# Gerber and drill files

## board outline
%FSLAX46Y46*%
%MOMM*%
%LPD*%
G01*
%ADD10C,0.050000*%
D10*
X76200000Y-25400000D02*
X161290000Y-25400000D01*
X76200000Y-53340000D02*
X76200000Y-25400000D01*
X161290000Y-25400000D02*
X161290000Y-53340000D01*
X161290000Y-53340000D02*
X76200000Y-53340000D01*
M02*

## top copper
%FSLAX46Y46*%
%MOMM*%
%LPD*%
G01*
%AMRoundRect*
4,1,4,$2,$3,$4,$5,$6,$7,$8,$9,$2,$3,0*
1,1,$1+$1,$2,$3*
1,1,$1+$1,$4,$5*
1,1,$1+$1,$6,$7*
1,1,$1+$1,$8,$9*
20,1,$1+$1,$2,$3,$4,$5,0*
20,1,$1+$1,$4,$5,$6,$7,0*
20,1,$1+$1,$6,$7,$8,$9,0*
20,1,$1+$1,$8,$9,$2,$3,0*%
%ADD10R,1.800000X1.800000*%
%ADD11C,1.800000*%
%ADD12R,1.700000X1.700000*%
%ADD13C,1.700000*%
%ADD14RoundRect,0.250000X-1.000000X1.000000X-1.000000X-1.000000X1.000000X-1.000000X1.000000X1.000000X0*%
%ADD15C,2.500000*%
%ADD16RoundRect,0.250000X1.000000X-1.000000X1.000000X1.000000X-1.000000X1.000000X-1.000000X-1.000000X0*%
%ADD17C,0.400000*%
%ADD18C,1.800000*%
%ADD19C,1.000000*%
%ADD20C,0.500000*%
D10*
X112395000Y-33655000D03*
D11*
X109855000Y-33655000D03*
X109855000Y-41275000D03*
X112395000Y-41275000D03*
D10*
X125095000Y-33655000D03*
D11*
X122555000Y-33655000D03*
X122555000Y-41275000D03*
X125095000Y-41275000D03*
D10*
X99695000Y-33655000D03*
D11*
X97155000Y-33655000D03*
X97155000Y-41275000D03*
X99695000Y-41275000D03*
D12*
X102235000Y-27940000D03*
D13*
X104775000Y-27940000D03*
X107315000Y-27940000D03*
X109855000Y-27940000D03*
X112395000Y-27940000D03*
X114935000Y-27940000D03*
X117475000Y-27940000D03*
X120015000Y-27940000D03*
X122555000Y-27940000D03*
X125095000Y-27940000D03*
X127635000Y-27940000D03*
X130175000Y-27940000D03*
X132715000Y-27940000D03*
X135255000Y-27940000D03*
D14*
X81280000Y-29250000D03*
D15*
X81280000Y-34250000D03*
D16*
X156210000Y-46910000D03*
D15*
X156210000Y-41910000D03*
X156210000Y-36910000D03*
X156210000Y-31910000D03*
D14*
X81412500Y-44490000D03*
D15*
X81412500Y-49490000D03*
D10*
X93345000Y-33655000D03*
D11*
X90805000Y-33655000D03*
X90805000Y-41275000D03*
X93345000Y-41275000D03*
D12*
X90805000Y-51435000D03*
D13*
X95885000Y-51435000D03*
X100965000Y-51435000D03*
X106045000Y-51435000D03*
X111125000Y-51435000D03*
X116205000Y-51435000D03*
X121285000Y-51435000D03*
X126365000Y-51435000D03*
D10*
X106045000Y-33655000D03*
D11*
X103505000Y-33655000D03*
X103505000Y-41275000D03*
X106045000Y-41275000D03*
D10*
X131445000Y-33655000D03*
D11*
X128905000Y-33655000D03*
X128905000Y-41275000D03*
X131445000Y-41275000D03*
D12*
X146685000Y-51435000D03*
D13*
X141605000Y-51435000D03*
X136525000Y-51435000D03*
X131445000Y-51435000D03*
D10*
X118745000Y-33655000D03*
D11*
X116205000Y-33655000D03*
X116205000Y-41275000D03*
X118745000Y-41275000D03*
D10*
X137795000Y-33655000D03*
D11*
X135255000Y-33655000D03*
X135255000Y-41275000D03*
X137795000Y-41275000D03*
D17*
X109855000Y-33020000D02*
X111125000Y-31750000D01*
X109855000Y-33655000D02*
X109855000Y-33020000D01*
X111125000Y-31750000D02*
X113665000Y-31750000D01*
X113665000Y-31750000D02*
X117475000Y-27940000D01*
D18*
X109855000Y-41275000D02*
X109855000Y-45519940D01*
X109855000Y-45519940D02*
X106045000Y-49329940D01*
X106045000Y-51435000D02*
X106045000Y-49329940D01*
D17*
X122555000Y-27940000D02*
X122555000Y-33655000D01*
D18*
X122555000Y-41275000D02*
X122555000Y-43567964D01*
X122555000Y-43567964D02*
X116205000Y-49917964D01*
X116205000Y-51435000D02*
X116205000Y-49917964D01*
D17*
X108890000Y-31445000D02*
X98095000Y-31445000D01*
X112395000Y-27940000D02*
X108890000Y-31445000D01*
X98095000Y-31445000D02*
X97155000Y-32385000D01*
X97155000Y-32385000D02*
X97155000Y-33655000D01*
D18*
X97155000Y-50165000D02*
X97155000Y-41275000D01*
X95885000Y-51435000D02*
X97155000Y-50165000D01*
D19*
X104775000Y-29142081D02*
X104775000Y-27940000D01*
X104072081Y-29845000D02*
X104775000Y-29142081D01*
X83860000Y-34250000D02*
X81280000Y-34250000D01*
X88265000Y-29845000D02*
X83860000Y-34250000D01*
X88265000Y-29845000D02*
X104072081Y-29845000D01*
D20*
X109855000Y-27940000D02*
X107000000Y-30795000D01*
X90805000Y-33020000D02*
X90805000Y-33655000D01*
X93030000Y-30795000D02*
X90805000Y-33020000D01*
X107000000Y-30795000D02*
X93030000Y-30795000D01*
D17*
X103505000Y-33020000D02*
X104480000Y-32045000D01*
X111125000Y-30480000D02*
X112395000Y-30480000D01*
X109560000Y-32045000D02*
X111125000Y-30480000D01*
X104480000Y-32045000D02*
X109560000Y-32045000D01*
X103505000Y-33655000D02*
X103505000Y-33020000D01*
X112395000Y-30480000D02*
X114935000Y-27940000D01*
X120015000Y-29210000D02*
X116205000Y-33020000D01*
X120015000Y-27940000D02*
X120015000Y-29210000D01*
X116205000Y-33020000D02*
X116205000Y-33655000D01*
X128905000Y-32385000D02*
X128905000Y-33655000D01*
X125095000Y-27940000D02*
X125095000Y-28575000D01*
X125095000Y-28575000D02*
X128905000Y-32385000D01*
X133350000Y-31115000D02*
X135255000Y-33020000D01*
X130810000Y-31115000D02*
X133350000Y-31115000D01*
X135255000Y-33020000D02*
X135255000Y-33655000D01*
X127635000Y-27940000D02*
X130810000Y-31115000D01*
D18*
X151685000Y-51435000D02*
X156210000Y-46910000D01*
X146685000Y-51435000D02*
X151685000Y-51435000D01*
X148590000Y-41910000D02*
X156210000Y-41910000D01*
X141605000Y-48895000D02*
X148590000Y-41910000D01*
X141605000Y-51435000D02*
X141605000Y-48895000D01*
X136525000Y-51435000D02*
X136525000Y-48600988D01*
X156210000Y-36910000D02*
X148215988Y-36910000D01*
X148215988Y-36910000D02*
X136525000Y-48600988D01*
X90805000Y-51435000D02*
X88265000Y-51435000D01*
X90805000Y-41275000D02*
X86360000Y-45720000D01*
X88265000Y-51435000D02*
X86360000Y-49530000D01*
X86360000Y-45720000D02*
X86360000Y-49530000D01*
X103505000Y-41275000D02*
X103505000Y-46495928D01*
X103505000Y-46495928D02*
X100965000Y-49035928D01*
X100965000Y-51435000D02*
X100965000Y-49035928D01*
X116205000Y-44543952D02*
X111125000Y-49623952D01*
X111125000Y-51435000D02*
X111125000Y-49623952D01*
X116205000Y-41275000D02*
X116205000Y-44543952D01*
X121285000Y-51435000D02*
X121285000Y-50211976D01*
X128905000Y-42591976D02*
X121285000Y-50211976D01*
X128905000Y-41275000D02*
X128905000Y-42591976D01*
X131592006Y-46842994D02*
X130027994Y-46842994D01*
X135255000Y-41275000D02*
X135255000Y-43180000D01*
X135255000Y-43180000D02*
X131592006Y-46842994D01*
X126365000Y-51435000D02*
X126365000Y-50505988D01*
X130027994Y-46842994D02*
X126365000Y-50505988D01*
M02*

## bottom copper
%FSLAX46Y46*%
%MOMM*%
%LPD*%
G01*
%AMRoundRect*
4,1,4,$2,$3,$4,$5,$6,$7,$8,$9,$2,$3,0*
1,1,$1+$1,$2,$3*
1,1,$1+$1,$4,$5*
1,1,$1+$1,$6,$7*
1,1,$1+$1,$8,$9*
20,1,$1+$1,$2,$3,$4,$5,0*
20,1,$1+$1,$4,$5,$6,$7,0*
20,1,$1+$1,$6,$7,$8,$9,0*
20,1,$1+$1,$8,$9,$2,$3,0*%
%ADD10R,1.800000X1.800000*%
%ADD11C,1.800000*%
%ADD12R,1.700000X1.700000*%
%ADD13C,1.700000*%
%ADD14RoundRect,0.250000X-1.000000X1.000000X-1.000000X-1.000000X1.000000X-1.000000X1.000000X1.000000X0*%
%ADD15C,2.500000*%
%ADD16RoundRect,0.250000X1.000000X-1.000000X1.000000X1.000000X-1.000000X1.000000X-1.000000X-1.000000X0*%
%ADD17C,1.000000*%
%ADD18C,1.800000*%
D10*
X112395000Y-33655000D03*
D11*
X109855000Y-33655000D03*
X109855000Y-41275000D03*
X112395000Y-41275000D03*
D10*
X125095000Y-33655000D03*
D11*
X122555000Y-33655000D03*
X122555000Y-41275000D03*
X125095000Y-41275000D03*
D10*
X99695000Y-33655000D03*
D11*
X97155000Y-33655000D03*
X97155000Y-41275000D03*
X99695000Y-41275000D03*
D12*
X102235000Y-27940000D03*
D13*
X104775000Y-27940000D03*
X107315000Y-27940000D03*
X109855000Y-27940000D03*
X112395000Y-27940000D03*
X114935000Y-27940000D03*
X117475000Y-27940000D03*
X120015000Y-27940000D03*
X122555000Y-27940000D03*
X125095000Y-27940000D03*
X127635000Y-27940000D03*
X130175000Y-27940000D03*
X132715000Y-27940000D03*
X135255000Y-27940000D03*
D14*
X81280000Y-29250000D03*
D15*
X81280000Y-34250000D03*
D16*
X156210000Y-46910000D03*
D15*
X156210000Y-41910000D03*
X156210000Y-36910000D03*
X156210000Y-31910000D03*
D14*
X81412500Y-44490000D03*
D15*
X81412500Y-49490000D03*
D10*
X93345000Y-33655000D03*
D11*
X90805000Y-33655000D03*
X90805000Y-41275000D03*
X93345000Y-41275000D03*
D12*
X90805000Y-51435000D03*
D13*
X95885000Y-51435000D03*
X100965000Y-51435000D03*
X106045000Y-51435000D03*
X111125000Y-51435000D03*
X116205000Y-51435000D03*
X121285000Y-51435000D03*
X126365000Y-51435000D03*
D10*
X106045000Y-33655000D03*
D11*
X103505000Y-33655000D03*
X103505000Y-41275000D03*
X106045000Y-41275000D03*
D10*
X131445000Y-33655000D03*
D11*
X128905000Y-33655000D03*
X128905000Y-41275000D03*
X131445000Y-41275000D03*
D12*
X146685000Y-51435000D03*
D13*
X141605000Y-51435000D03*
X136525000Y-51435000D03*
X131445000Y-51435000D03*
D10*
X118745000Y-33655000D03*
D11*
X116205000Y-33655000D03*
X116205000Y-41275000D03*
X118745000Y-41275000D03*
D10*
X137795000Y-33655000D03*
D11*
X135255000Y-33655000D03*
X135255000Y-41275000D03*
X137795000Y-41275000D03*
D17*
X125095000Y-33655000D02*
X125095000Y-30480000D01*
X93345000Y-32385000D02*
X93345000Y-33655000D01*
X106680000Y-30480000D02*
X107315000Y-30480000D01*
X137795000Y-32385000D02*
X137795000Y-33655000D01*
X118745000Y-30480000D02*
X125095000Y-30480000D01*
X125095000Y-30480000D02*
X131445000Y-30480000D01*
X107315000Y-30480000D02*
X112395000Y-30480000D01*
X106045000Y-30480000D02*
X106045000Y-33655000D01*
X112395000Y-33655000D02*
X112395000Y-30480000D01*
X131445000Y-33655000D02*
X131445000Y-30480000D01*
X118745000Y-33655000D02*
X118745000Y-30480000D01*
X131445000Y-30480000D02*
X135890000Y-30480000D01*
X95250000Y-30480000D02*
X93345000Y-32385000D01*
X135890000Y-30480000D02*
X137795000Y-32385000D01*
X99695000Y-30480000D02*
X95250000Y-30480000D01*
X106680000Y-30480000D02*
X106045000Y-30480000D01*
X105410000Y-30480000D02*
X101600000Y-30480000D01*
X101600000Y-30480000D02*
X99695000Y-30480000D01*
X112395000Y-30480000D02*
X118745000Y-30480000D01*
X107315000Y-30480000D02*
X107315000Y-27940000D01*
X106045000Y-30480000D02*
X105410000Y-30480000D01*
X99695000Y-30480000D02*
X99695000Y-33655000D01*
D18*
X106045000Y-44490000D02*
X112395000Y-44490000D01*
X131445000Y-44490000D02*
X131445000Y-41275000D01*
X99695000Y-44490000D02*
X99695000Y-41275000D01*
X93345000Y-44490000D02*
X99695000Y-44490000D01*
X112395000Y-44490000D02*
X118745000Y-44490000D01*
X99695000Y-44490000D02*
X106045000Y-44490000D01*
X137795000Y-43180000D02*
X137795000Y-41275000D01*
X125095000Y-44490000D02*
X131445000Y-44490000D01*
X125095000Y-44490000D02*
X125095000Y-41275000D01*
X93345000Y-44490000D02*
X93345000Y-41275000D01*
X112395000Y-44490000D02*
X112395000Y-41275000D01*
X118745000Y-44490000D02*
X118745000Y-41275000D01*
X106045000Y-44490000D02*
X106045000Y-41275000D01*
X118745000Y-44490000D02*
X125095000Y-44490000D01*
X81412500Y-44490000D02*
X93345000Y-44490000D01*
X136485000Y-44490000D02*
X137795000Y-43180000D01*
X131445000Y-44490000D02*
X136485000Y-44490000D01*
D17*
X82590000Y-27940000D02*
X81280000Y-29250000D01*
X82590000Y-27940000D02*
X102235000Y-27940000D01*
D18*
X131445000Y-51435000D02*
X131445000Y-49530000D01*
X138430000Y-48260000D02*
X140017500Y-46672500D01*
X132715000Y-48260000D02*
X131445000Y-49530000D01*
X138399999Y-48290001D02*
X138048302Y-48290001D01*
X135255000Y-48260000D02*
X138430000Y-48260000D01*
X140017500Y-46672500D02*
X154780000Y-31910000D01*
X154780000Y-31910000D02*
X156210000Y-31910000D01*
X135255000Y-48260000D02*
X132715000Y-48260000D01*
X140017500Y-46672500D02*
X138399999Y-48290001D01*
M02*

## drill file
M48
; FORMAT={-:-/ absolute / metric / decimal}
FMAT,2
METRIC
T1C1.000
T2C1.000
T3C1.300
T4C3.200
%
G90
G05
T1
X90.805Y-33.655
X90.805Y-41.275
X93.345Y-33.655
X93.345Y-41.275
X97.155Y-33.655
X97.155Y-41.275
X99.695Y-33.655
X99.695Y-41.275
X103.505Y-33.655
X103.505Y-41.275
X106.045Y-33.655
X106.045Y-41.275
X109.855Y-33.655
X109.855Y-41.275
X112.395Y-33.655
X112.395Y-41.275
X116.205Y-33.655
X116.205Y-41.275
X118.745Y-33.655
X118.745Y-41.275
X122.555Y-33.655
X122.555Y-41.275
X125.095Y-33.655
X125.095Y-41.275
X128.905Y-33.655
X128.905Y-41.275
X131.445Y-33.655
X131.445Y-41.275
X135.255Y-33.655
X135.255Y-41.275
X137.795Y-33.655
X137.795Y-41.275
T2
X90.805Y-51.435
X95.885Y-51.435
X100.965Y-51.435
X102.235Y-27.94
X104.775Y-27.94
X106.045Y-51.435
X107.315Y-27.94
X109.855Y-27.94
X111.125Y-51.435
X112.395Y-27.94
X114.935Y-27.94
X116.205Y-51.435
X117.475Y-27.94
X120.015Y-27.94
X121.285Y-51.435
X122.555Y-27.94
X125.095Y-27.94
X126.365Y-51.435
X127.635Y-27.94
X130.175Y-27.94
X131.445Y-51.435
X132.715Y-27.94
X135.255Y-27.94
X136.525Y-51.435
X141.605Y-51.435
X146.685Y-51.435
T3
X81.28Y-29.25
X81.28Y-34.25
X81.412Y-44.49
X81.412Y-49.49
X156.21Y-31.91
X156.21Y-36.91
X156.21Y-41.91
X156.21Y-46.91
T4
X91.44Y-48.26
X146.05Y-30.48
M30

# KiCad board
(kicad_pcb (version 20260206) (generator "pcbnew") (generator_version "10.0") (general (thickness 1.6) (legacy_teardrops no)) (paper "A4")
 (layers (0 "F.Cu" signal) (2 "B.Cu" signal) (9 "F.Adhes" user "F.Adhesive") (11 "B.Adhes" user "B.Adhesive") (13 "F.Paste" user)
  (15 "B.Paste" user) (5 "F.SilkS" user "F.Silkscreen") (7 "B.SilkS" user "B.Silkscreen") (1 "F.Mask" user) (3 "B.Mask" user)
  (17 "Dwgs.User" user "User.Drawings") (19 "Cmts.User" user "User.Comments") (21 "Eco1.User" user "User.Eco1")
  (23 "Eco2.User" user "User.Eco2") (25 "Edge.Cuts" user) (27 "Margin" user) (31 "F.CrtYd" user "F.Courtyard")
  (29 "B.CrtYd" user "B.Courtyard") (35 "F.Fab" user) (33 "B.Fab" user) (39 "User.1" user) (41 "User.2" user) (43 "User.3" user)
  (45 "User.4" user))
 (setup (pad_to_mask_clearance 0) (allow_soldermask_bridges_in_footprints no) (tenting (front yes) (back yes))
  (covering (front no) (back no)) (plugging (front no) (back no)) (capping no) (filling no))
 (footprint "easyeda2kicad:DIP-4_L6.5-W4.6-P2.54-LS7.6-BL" (layer "F.Cu") (at 111.125 37.465 180)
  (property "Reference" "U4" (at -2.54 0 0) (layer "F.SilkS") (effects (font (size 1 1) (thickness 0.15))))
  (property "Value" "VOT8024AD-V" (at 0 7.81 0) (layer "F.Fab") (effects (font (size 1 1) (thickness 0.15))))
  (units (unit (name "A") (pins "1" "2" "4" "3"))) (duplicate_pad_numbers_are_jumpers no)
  (pad "1" thru_hole rect (at -1.27 3.81) (size 1.8 1.8) (drill 0.999998) (layers "*.Cu" "*.Mask") (remove_unused_layers no) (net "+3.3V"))
  (pad "2" thru_hole circle (at 1.27 3.81 270) (size 1.8 1.8) (drill 0.999998) (layers "*.Cu" "*.Mask") (remove_unused_layers no)
   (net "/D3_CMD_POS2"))
  (pad "3" thru_hole circle (at 1.27 -3.81 270) (size 1.8 1.8) (drill 0.999998) (layers "*.Cu" "*.Mask") (remove_unused_layers no)
   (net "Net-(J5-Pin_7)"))
  (pad "4" thru_hole circle (at -1.27 -3.81 270) (size 1.8 1.8) (drill 0.999998) (layers "*.Cu" "*.Mask") (remove_unused_layers no)
   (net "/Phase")))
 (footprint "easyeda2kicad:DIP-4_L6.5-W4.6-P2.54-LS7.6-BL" (layer "F.Cu") (at 123.825 37.465 180)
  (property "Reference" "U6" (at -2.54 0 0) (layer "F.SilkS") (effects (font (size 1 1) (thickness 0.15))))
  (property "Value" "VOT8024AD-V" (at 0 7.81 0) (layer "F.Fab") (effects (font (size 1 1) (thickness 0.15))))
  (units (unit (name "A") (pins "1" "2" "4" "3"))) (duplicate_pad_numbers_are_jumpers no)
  (pad "1" thru_hole rect (at -1.27 3.81) (size 1.8 1.8) (drill 0.999998) (layers "*.Cu" "*.Mask") (remove_unused_layers no) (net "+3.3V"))
  (pad "2" thru_hole circle (at 1.27 3.81 270) (size 1.8 1.8) (drill 0.999998) (layers "*.Cu" "*.Mask") (remove_unused_layers no)
   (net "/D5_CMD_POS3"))
  (pad "3" thru_hole circle (at 1.27 -3.81 270) (size 1.8 1.8) (drill 0.999998) (layers "*.Cu" "*.Mask") (remove_unused_layers no)
   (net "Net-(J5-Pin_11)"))
  (pad "4" thru_hole circle (at -1.27 -3.81 270) (size 1.8 1.8) (drill 0.999998) (layers "*.Cu" "*.Mask") (remove_unused_layers no)
   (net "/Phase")))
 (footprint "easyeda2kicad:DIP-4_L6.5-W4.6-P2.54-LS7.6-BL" (layer "F.Cu") (at 98.425 37.465 180)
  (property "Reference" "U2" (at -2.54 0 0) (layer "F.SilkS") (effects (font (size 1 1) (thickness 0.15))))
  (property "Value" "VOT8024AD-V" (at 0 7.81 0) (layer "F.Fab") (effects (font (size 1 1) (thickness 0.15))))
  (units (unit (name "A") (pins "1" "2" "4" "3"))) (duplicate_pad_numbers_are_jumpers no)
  (pad "1" thru_hole rect (at -1.27 3.81) (size 1.8 1.8) (drill 0.999998) (layers "*.Cu" "*.Mask") (remove_unused_layers no) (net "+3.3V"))
  (pad "2" thru_hole circle (at 1.27 3.81 270) (size 1.8 1.8) (drill 0.999998) (layers "*.Cu" "*.Mask") (remove_unused_layers no)
   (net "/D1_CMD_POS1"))
  (pad "3" thru_hole circle (at 1.27 -3.81 270) (size 1.8 1.8) (drill 0.999998) (layers "*.Cu" "*.Mask") (remove_unused_layers no)
   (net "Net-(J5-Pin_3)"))
  (pad "4" thru_hole circle (at -1.27 -3.81 270) (size 1.8 1.8) (drill 0.999998) (layers "*.Cu" "*.Mask") (remove_unused_layers no)
   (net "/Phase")))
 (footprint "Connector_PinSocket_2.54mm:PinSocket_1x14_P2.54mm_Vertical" (layer "F.Cu") (at 102.235 27.94 90)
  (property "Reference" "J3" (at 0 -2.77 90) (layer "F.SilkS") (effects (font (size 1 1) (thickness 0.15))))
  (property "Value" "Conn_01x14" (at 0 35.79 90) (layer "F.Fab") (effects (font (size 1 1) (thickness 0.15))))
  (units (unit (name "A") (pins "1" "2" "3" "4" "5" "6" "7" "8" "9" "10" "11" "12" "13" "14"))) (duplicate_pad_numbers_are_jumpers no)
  (pad "1" thru_hole rect (at 0 0 90) (size 1.7 1.7) (drill 1) (layers "*.Cu" "*.Mask") (remove_unused_layers no) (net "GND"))
  (pad "2" thru_hole circle (at 0 2.54 90) (size 1.7 1.7) (drill 1) (layers "*.Cu" "*.Mask") (remove_unused_layers no) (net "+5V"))
  (pad "3" thru_hole circle (at 0 5.08 90) (size 1.7 1.7) (drill 1) (layers "*.Cu" "*.Mask") (remove_unused_layers no) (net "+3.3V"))
  (pad "4" thru_hole circle (at 0 7.62 90) (size 1.7 1.7) (drill 1) (layers "*.Cu" "*.Mask") (remove_unused_layers no) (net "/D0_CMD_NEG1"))
  (pad "5" thru_hole circle (at 0 10.16 90) (size 1.7 1.7) (drill 1) (layers "*.Cu" "*.Mask") (remove_unused_layers no) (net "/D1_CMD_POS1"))
  (pad "6" thru_hole circle (at 0 12.7 90) (size 1.7 1.7) (drill 1) (layers "*.Cu" "*.Mask") (remove_unused_layers no) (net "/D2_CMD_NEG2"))
  (pad "7" thru_hole circle (at 0 15.24 90) (size 1.7 1.7) (drill 1) (layers "*.Cu" "*.Mask") (remove_unused_layers no) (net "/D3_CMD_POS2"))
  (pad "8" thru_hole circle (at 0 17.78 90) (size 1.7 1.7) (drill 1) (layers "*.Cu" "*.Mask") (remove_unused_layers no) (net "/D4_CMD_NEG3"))
  (pad "9" thru_hole circle (at 0 20.32 90) (size 1.7 1.7) (drill 1) (layers "*.Cu" "*.Mask") (remove_unused_layers no) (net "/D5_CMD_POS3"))
  (pad "10" thru_hole circle (at 0 22.86 90) (size 1.7 1.7) (drill 1) (layers "*.Cu" "*.Mask") (remove_unused_layers no)
   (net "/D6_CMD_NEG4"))
  (pad "11" thru_hole circle (at 0 25.4 90) (size 1.7 1.7) (drill 1) (layers "*.Cu" "*.Mask") (remove_unused_layers no) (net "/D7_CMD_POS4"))
  (pad "12" thru_hole circle (at 0 27.94 90) (size 1.7 1.7) (drill 1) (layers "*.Cu" "*.Mask") (remove_unused_layers no)
   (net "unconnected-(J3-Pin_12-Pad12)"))
  (pad "13" thru_hole circle (at 0 30.48 90) (size 1.7 1.7) (drill 1) (layers "*.Cu" "*.Mask") (remove_unused_layers no)
   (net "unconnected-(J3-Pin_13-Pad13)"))
  (pad "14" thru_hole circle (at 0 33.02 90) (size 1.7 1.7) (drill 1) (layers "*.Cu" "*.Mask") (remove_unused_layers no)
   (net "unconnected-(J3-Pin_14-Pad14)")))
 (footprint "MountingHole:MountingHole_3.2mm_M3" (layer "F.Cu") (at 91.44 48.26)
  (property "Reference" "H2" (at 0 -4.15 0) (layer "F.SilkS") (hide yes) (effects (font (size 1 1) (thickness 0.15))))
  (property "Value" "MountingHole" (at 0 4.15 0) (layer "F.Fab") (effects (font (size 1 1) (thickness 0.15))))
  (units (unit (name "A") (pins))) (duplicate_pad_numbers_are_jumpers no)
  (pad "" np_thru_hole circle (at 0 0) (size 3.2 3.2) (drill 3.2) (layers "*.Cu" "*.Mask")))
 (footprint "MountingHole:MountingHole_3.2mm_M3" (layer "F.Cu") (at 146.05 30.48)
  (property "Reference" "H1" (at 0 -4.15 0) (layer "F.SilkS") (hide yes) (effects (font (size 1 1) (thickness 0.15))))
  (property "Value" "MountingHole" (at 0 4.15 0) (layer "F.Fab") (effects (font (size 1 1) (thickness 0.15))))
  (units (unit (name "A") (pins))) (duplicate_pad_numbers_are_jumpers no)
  (pad "" np_thru_hole circle (at 0 0) (size 3.2 3.2) (drill 3.2) (layers "*.Cu" "*.Mask")))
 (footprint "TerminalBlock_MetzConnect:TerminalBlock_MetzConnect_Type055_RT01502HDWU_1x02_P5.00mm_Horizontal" (layer "F.Cu")
  (at 81.28 29.25 -90)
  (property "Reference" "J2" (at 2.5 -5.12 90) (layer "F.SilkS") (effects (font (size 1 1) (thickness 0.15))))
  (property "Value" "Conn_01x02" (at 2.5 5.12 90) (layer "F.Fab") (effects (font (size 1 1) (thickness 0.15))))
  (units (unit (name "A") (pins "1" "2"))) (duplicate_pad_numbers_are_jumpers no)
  (pad "1" thru_hole roundrect (at 0 0 270) (size 2.5 2.5) (drill 1.3) (layers "*.Cu" "*.Mask") (remove_unused_layers no)
   (roundrect_rratio 0.1) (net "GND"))
  (pad "2" thru_hole circle (at 5 0 270) (size 2.5 2.5) (drill 1.3) (layers "*.Cu" "*.Mask") (remove_unused_layers no) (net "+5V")))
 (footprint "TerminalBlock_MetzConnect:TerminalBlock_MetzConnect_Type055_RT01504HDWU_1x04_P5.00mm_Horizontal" (layer "F.Cu")
  (at 156.21 46.91 90)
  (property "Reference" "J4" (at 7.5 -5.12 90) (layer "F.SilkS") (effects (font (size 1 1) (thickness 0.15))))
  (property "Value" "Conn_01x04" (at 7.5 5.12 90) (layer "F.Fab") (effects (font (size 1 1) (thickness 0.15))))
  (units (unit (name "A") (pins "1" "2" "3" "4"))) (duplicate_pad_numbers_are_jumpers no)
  (pad "1" thru_hole roundrect (at 0 0 90) (size 2.5 2.5) (drill 1.3) (layers "*.Cu" "*.Mask") (remove_unused_layers no)
   (roundrect_rratio 0.1) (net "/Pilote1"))
  (pad "2" thru_hole circle (at 5 0 90) (size 2.5 2.5) (drill 1.3) (layers "*.Cu" "*.Mask") (remove_unused_layers no) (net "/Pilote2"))
  (pad "3" thru_hole circle (at 10 0 90) (size 2.5 2.5) (drill 1.3) (layers "*.Cu" "*.Mask") (remove_unused_layers no) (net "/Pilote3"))
  (pad "4" thru_hole circle (at 15 0 90) (size 2.5 2.5) (drill 1.3) (layers "*.Cu" "*.Mask") (remove_unused_layers no) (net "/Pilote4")))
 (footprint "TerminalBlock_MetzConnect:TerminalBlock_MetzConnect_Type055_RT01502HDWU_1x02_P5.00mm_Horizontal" (layer "F.Cu")
  (at 81.4125 44.49 -90)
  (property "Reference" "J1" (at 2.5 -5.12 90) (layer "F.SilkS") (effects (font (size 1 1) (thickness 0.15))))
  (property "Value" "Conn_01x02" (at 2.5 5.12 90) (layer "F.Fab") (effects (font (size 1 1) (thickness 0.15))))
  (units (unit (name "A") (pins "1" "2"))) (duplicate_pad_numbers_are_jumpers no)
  (pad "1" thru_hole roundrect (at 0 0 270) (size 2.5 2.5) (drill 1.3) (layers "*.Cu" "*.Mask") (remove_unused_layers no)
   (roundrect_rratio 0.1) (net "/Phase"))
  (pad "2" thru_hole circle (at 5 0 270) (size 2.5 2.5) (drill 1.3) (layers "*.Cu" "*.Mask") (remove_unused_layers no)
   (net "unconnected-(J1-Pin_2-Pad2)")))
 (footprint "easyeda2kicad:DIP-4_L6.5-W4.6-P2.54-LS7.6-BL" (layer "F.Cu") (at 92.075 37.465 180)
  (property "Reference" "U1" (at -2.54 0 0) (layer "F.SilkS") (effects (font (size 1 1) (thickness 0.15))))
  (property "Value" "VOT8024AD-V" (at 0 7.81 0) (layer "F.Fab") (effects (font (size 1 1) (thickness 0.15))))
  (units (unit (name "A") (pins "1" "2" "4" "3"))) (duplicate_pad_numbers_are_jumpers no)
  (pad "1" thru_hole rect (at -1.27 3.81) (size 1.8 1.8) (drill 0.999998) (layers "*.Cu" "*.Mask") (remove_unused_layers no) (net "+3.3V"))
  (pad "2" thru_hole circle (at 1.27 3.81 270) (size 1.8 1.8) (drill 0.999998) (layers "*.Cu" "*.Mask") (remove_unused_layers no)
   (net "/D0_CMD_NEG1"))
  (pad "3" thru_hole circle (at 1.27 -3.81 270) (size 1.8 1.8) (drill 0.999998) (layers "*.Cu" "*.Mask") (remove_unused_layers no)
   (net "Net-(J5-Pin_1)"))
  (pad "4" thru_hole circle (at -1.27 -3.81 270) (size 1.8 1.8) (drill 0.999998) (layers "*.Cu" "*.Mask") (remove_unused_layers no)
   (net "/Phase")))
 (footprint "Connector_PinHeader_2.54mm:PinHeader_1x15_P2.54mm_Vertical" (layer "F.Cu") (at 90.805 51.435 90)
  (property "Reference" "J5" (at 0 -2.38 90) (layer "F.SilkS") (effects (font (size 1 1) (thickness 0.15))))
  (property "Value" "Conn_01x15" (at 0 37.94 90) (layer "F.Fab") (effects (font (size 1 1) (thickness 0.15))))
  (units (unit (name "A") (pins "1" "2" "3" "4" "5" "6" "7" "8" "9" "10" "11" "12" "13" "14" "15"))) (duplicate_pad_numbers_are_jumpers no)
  (pad "1" thru_hole rect (at 0 0 90) (size 1.7 1.7) (drill 1) (layers "*.Cu" "*.Mask") (remove_unused_layers no) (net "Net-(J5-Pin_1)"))
  (pad "3" thru_hole circle (at 0 5.08 90) (size 1.7 1.7) (drill 1) (layers "*.Cu" "*.Mask") (remove_unused_layers no)
   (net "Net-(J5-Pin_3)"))
  (pad "5" thru_hole circle (at 0 10.16 90) (size 1.7 1.7) (drill 1) (layers "*.Cu" "*.Mask") (remove_unused_layers no)
   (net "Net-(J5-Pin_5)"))
  (pad "7" thru_hole circle (at 0 15.24 90) (size 1.7 1.7) (drill 1) (layers "*.Cu" "*.Mask") (remove_unused_layers no)
   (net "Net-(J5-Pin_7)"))
  (pad "9" thru_hole circle (at 0 20.32 90) (size 1.7 1.7) (drill 1) (layers "*.Cu" "*.Mask") (remove_unused_layers no)
   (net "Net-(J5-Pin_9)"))
  (pad "11" thru_hole circle (at 0 25.4 90) (size 1.7 1.7) (drill 1) (layers "*.Cu" "*.Mask") (remove_unused_layers no)
   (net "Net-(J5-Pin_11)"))
  (pad "13" thru_hole circle (at 0 30.48 90) (size 1.7 1.7) (drill 1) (layers "*.Cu" "*.Mask") (remove_unused_layers no)
   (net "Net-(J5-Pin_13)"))
  (pad "15" thru_hole circle (at 0 35.56 90) (size 1.7 1.7) (drill 1) (layers "*.Cu" "*.Mask") (remove_unused_layers no)
   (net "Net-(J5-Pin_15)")))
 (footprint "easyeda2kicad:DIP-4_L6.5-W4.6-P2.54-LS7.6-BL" (layer "F.Cu") (at 104.775 37.465 180)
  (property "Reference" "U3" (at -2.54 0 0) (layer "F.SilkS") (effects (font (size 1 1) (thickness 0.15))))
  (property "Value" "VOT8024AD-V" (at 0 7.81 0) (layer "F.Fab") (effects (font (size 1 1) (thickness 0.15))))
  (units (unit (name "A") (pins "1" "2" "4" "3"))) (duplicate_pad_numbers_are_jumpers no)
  (pad "1" thru_hole rect (at -1.27 3.81) (size 1.8 1.8) (drill 0.999998) (layers "*.Cu" "*.Mask") (remove_unused_layers no) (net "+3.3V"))
  (pad "2" thru_hole circle (at 1.27 3.81 270) (size 1.8 1.8) (drill 0.999998) (layers "*.Cu" "*.Mask") (remove_unused_layers no)
   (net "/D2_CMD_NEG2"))
  (pad "3" thru_hole circle (at 1.27 -3.81 270) (size 1.8 1.8) (drill 0.999998) (layers "*.Cu" "*.Mask") (remove_unused_layers no)
   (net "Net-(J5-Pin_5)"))
  (pad "4" thru_hole circle (at -1.27 -3.81 270) (size 1.8 1.8) (drill 0.999998) (layers "*.Cu" "*.Mask") (remove_unused_layers no)
   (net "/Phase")))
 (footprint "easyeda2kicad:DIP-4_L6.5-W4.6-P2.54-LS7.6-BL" (layer "F.Cu") (at 130.175 37.465 180)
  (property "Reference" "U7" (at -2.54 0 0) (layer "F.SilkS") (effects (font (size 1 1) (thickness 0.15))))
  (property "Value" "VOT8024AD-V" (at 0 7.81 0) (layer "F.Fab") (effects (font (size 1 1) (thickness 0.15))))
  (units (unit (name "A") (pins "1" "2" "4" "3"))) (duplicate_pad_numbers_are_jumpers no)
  (pad "1" thru_hole rect (at -1.27 3.81) (size 1.8 1.8) (drill 0.999998) (layers "*.Cu" "*.Mask") (remove_unused_layers no) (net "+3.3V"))
  (pad "2" thru_hole circle (at 1.27 3.81 270) (size 1.8 1.8) (drill 0.999998) (layers "*.Cu" "*.Mask") (remove_unused_layers no)
   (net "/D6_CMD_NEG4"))
  (pad "3" thru_hole circle (at 1.27 -3.81 270) (size 1.8 1.8) (drill 0.999998) (layers "*.Cu" "*.Mask") (remove_unused_layers no)
   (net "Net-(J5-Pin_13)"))
  (pad "4" thru_hole circle (at -1.27 -3.81 270) (size 1.8 1.8) (drill 0.999998) (layers "*.Cu" "*.Mask") (remove_unused_layers no)
   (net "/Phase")))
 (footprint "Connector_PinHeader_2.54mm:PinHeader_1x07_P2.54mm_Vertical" (layer "F.Cu") (at 146.685 51.435 -90)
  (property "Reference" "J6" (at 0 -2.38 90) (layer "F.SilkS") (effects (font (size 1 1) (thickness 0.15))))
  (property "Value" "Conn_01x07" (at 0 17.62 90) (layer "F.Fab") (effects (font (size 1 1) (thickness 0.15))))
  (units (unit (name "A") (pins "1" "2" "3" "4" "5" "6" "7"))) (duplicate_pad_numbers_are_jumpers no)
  (pad "1" thru_hole rect (at 0 0 270) (size 1.7 1.7) (drill 1) (layers "*.Cu" "*.Mask") (remove_unused_layers no) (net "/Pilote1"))
  (pad "3" thru_hole circle (at 0 5.08 270) (size 1.7 1.7) (drill 1) (layers "*.Cu" "*.Mask") (remove_unused_layers no) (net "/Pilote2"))
  (pad "5" thru_hole circle (at 0 10.16 270) (size 1.7 1.7) (drill 1) (layers "*.Cu" "*.Mask") (remove_unused_layers no) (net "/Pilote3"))
  (pad "7" thru_hole circle (at 0 15.24 270) (size 1.7 1.7) (drill 1) (layers "*.Cu" "*.Mask") (remove_unused_layers no) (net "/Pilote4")))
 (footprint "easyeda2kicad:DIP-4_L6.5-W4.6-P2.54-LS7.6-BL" (layer "F.Cu") (at 117.475 37.465 180)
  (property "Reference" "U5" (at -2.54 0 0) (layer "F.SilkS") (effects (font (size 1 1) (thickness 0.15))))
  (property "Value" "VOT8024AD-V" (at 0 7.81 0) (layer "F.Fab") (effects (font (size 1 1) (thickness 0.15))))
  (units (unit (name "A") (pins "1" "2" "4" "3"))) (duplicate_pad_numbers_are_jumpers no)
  (pad "1" thru_hole rect (at -1.27 3.81) (size 1.8 1.8) (drill 0.999998) (layers "*.Cu" "*.Mask") (remove_unused_layers no) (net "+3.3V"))
  (pad "2" thru_hole circle (at 1.27 3.81 270) (size 1.8 1.8) (drill 0.999998) (layers "*.Cu" "*.Mask") (remove_unused_layers no)
   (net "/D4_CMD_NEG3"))
  (pad "3" thru_hole circle (at 1.27 -3.81 270) (size 1.8 1.8) (drill 0.999998) (layers "*.Cu" "*.Mask") (remove_unused_layers no)
   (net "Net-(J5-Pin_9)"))
  (pad "4" thru_hole circle (at -1.27 -3.81 270) (size 1.8 1.8) (drill 0.999998) (layers "*.Cu" "*.Mask") (remove_unused_layers no)
   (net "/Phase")))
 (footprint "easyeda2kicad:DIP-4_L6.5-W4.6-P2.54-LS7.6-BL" (layer "F.Cu") (at 136.525 37.465 180)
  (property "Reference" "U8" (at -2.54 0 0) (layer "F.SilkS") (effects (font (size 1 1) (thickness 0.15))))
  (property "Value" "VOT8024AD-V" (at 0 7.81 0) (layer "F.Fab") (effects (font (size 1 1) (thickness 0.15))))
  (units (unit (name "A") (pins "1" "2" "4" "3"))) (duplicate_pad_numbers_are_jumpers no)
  (pad "1" thru_hole rect (at -1.27 3.81) (size 1.8 1.8) (drill 0.999998) (layers "*.Cu" "*.Mask") (remove_unused_layers no) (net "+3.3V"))
  (pad "2" thru_hole circle (at 1.27 3.81 270) (size 1.8 1.8) (drill 0.999998) (layers "*.Cu" "*.Mask") (remove_unused_layers no)
   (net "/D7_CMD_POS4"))
  (pad "3" thru_hole circle (at 1.27 -3.81 270) (size 1.8 1.8) (drill 0.999998) (layers "*.Cu" "*.Mask") (remove_unused_layers no)
   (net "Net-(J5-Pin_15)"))
  (pad "4" thru_hole circle (at -1.27 -3.81 270) (size 1.8 1.8) (drill 0.999998) (layers "*.Cu" "*.Mask") (remove_unused_layers no)
   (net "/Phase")))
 (gr_line (start 76.2 25.4) (end 161.29 25.4) (stroke (width 0.05) (type default)) (layer "Edge.Cuts"))
 (gr_line (start 76.2 53.34) (end 76.2 25.4) (stroke (width 0.05) (type default)) (layer "Edge.Cuts"))
 (gr_line (start 161.29 25.4) (end 161.29 53.34) (stroke (width 0.05) (type default)) (layer "Edge.Cuts"))
 (gr_line (start 161.29 53.34) (end 76.2 53.34) (stroke (width 0.05) (type default)) (layer "Edge.Cuts"))
 (segment (start 125.095 33.655) (end 125.095 30.48) (width 1) (layer "B.Cu") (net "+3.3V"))
 (segment (start 93.345 32.385) (end 93.345 33.655) (width 1) (layer "B.Cu") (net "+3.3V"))
 (segment (start 106.68 30.48) (end 107.315 30.48) (width 1) (layer "B.Cu") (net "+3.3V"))
 (segment (start 137.795 32.385) (end 137.795 33.655) (width 1) (layer "B.Cu") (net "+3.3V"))
 (segment (start 118.745 30.48) (end 125.095 30.48) (width 1) (layer "B.Cu") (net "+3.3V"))
 (segment (start 125.095 30.48) (end 131.445 30.48) (width 1) (layer "B.Cu") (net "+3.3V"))
 (segment (start 107.315 30.48) (end 112.395 30.48) (width 1) (layer "B.Cu") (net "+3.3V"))
 (segment (start 106.045 30.48) (end 106.045 33.655) (width 1) (layer "B.Cu") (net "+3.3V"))
 (segment (start 112.395 33.655) (end 112.395 30.48) (width 1) (layer "B.Cu") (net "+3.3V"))
 (segment (start 131.445 33.655) (end 131.445 30.48) (width 1) (layer "B.Cu") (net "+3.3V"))
 (segment (start 118.745 33.655) (end 118.745 30.48) (width 1) (layer "B.Cu") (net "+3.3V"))
 (segment (start 131.445 30.48) (end 135.89 30.48) (width 1) (layer "B.Cu") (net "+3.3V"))
 (segment (start 95.25 30.48) (end 93.345 32.385) (width 1) (layer "B.Cu") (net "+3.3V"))
 (segment (start 135.89 30.48) (end 137.795 32.385) (width 1) (layer "B.Cu") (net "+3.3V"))
 (segment (start 99.695 30.48) (end 95.25 30.48) (width 1) (layer "B.Cu") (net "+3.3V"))
 (segment (start 106.68 30.48) (end 106.045 30.48) (width 1) (layer "B.Cu") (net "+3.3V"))
 (segment (start 105.41 30.48) (end 101.6 30.48) (width 1) (layer "B.Cu") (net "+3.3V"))
 (segment (start 101.6 30.48) (end 99.695 30.48) (width 1) (layer "B.Cu") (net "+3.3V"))
 (segment (start 112.395 30.48) (end 118.745 30.48) (width 1) (layer "B.Cu") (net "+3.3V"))
 (segment (start 107.315 30.48) (end 107.315 27.94) (width 1) (layer "B.Cu") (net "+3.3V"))
 (segment (start 106.045 30.48) (end 105.41 30.48) (width 1) (layer "B.Cu") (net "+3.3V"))
 (segment (start 99.695 30.48) (end 99.695 33.655) (width 1) (layer "B.Cu") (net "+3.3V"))
 (segment (start 109.855 33.02) (end 111.125 31.75) (width 0.4) (layer "F.Cu") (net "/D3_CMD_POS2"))
 (segment (start 109.855 33.655) (end 109.855 33.02) (width 0.4) (layer "F.Cu") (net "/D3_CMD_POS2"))
 (segment (start 111.125 31.75) (end 113.665 31.75) (width 0.4) (layer "F.Cu") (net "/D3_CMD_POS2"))
 (segment (start 113.665 31.75) (end 117.475 27.94) (width 0.4) (layer "F.Cu") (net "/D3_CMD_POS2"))
 (segment (start 109.855 41.275) (end 109.855 45.51994) (width 1.8) (layer "F.Cu") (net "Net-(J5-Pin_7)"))
 (segment (start 109.855 45.51994) (end 106.045 49.32994) (width 1.8) (layer "F.Cu") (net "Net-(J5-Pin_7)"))
 (segment (start 106.045 51.435) (end 106.045 49.32994) (width 1.8) (layer "F.Cu") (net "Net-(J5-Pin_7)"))
 (segment (start 106.045 44.49) (end 112.395 44.49) (width 1.8) (layer "B.Cu") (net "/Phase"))
 (segment (start 131.445 44.49) (end 131.445 41.275) (width 1.8) (layer "B.Cu") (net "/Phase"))
 (segment (start 99.695 44.49) (end 99.695 41.275) (width 1.8) (layer "B.Cu") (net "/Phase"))
 (segment (start 93.345 44.49) (end 99.695 44.49) (width 1.8) (layer "B.Cu") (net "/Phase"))
 (segment (start 112.395 44.49) (end 118.745 44.49) (width 1.8) (layer "B.Cu") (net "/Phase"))
 (segment (start 99.695 44.49) (end 106.045 44.49) (width 1.8) (layer "B.Cu") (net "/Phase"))
 (segment (start 137.795 43.18) (end 137.795 41.275) (width 1.8) (layer "B.Cu") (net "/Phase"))
 (segment (start 125.095 44.49) (end 131.445 44.49) (width 1.8) (layer "B.Cu") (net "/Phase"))
 (segment (start 125.095 44.49) (end 125.095 41.275) (width 1.8) (layer "B.Cu") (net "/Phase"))
 (segment (start 93.345 44.49) (end 93.345 41.275) (width 1.8) (layer "B.Cu") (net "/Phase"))
 (segment (start 112.395 44.49) (end 112.395 41.275) (width 1.8) (layer "B.Cu") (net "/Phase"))
 (segment (start 118.745 44.49) (end 118.745 41.275) (width 1.8) (layer "B.Cu") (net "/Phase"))
 (segment (start 106.045 44.49) (end 106.045 41.275) (width 1.8) (layer "B.Cu") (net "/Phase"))
 (segment (start 118.745 44.49) (end 125.095 44.49) (width 1.8) (layer "B.Cu") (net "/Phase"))
 (segment (start 81.4125 44.49) (end 93.345 44.49) (width 1.8) (layer "B.Cu") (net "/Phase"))
 (segment (start 136.485 44.49) (end 137.795 43.18) (width 1.8) (layer "B.Cu") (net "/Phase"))
 (segment (start 131.445 44.49) (end 136.485 44.49) (width 1.8) (layer "B.Cu") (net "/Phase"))
 (segment (start 122.555 27.94) (end 122.555 33.655) (width 0.4) (layer "F.Cu") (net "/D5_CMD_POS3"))
 (segment (start 122.555 41.275) (end 122.555 43.567964) (width 1.8) (layer "F.Cu") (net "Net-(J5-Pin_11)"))
 (segment (start 122.555 43.567964) (end 116.205 49.917964) (width 1.8) (layer "F.Cu") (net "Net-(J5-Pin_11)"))
 (segment (start 116.205 51.435) (end 116.205 49.917964) (width 1.8) (layer "F.Cu") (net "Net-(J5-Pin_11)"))
 (segment (start 108.89 31.445) (end 98.095 31.445) (width 0.4) (layer "F.Cu") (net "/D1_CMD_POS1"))
 (segment (start 112.395 27.94) (end 108.89 31.445) (width 0.4) (layer "F.Cu") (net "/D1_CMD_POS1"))
 (segment (start 98.095 31.445) (end 97.155 32.385) (width 0.4) (layer "F.Cu") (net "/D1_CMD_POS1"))
 (segment (start 97.155 32.385) (end 97.155 33.655) (width 0.4) (layer "F.Cu") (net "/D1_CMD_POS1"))
 (segment (start 97.155 50.165) (end 97.155 41.275) (width 1.8) (layer "F.Cu") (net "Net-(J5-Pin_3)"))
 (segment (start 95.885 51.435) (end 97.155 50.165) (width 1.8) (layer "F.Cu") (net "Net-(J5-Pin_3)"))
 (segment (start 82.59 27.94) (end 81.28 29.25) (width 1) (layer "B.Cu") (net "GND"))
 (segment (start 82.59 27.94) (end 102.235 27.94) (width 1) (layer "B.Cu") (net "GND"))
 (segment (start 104.775 29.142081) (end 104.775 27.94) (width 1) (layer "F.Cu") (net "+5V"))
 (segment (start 104.072081 29.845) (end 104.775 29.142081) (width 1) (layer "F.Cu") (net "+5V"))
 (segment (start 83.86 34.25) (end 81.28 34.25) (width 1) (layer "F.Cu") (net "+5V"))
 (segment (start 88.265 29.845) (end 83.86 34.25) (width 1) (layer "F.Cu") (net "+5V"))
 (segment (start 88.265 29.845) (end 104.072081 29.845) (width 1) (layer "F.Cu") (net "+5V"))
 (segment (start 109.855 27.94) (end 107 30.795) (width 0.5) (layer "F.Cu") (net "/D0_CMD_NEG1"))
 (segment (start 90.805 33.02) (end 90.805 33.655) (width 0.5) (layer "F.Cu") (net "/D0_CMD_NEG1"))
 (segment (start 93.03 30.795) (end 90.805 33.02) (width 0.5) (layer "F.Cu") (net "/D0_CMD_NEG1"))
 (segment (start 107 30.795) (end 93.03 30.795) (width 0.5) (layer "F.Cu") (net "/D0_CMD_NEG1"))
 (segment (start 103.505 33.02) (end 104.48 32.045) (width 0.4) (layer "F.Cu") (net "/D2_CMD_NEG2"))
 (segment (start 111.125 30.48) (end 112.395 30.48) (width 0.4) (layer "F.Cu") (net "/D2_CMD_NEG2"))
 (segment (start 109.56 32.045) (end 111.125 30.48) (width 0.4) (layer "F.Cu") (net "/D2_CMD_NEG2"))
 (segment (start 104.48 32.045) (end 109.56 32.045) (width 0.4) (layer "F.Cu") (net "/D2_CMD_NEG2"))
 (segment (start 103.505 33.655) (end 103.505 33.02) (width 0.4) (layer "F.Cu") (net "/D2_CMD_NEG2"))
 (segment (start 112.395 30.48) (end 114.935 27.94) (width 0.4) (layer "F.Cu") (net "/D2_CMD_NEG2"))
 (segment (start 120.015 29.21) (end 116.205 33.02) (width 0.4) (layer "F.Cu") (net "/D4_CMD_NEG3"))
 (segment (start 120.015 27.94) (end 120.015 29.21) (width 0.4) (layer "F.Cu") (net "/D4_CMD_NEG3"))
 (segment (start 116.205 33.02) (end 116.205 33.655) (width 0.4) (layer "F.Cu") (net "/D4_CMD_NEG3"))
 (segment (start 128.905 32.385) (end 128.905 33.655) (width 0.4) (layer "F.Cu") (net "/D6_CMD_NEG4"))
 (segment (start 125.095 27.94) (end 125.095 28.575) (width 0.4) (layer "F.Cu") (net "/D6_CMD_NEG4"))
 (segment (start 125.095 28.575) (end 128.905 32.385) (width 0.4) (layer "F.Cu") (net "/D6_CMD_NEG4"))
 (segment (start 133.35 31.115) (end 135.255 33.02) (width 0.4) (layer "F.Cu") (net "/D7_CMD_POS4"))
 (segment (start 130.81 31.115) (end 133.35 31.115) (width 0.4) (layer "F.Cu") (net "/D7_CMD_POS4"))
 (segment (start 135.255 33.02) (end 135.255 33.655) (width 0.4) (layer "F.Cu") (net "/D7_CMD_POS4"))
 (segment (start 127.635 27.94) (end 130.81 31.115) (width 0.4) (layer "F.Cu") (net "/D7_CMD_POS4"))
 (segment (start 151.685 51.435) (end 156.21 46.91) (width 1.8) (layer "F.Cu") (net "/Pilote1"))
 (segment (start 146.685 51.435) (end 151.685 51.435) (width 1.8) (layer "F.Cu") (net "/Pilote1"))
 (segment (start 148.59 41.91) (end 156.21 41.91) (width 1.8) (layer "F.Cu") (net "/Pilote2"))
 (segment (start 141.605 48.895) (end 148.59 41.91) (width 1.8) (layer "F.Cu") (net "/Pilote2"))
 (segment (start 141.605 51.435) (end 141.605 48.895) (width 1.8) (layer "F.Cu") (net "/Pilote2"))
 (segment (start 136.525 51.435) (end 136.525 48.600988) (width 1.8) (layer "F.Cu") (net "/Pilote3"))
 (segment (start 156.21 36.91) (end 148.215988 36.91) (width 1.8) (layer "F.Cu") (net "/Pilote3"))
 (segment (start 148.215988 36.91) (end 136.525 48.600988) (width 1.8) (layer "F.Cu") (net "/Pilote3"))
 (segment (start 131.445 51.435) (end 131.445 49.53) (width 1.8) (layer "B.Cu") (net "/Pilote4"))
 (segment (start 138.43 48.26) (end 140.0175 46.6725) (width 1.8) (layer "B.Cu") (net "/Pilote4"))
 (segment (start 132.715 48.26) (end 131.445 49.53) (width 1.8) (layer "B.Cu") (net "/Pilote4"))
 (segment (start 138.399999 48.290001) (end 138.048302 48.290001) (width 1.8) (layer "B.Cu") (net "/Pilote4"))
 (segment (start 135.255 48.26) (end 138.43 48.26) (width 1.8) (layer "B.Cu") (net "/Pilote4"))
 (segment (start 140.0175 46.6725) (end 154.78 31.91) (width 1.8) (layer "B.Cu") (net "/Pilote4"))
 (segment (start 154.78 31.91) (end 156.21 31.91) (width 1.8) (layer "B.Cu") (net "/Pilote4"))
 (segment (start 135.255 48.26) (end 132.715 48.26) (width 1.8) (layer "B.Cu") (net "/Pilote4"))
 (segment (start 140.0175 46.6725) (end 138.399999 48.290001) (width 1.8) (layer "B.Cu") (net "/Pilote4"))
 (segment (start 90.805 51.435) (end 88.265 51.435) (width 1.8) (layer "F.Cu") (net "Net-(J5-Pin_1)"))
 (segment (start 90.805 41.275) (end 86.36 45.72) (width 1.8) (layer "F.Cu") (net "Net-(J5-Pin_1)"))
 (segment (start 88.265 51.435) (end 86.36 49.53) (width 1.8) (layer "F.Cu") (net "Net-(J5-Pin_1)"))
 (segment (start 86.36 45.72) (end 86.36 49.53) (width 1.8) (layer "F.Cu") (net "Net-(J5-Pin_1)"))
 (segment (start 103.505 41.275) (end 103.505 46.495928) (width 1.8) (layer "F.Cu") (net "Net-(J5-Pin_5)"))
 (segment (start 103.505 46.495928) (end 100.965 49.035928) (width 1.8) (layer "F.Cu") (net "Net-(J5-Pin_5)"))
 (segment (start 100.965 51.435) (end 100.965 49.035928) (width 1.8) (layer "F.Cu") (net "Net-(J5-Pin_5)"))
 (segment (start 116.205 44.543952) (end 111.125 49.623952) (width 1.8) (layer "F.Cu") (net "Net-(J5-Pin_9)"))
 (segment (start 111.125 51.435) (end 111.125 49.623952) (width 1.8) (layer "F.Cu") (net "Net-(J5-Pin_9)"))
 (segment (start 116.205 41.275) (end 116.205 44.543952) (width 1.8) (layer "F.Cu") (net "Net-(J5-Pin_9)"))
 (segment (start 121.285 51.435) (end 121.285 50.211976) (width 1.8) (layer "F.Cu") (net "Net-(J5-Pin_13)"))
 (segment (start 128.905 42.591976) (end 121.285 50.211976) (width 1.8) (layer "F.Cu") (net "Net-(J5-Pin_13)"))
 (segment (start 128.905 41.275) (end 128.905 42.591976) (width 1.8) (layer "F.Cu") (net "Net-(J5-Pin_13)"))
 (segment (start 131.592006 46.842994) (end 130.027994 46.842994) (width 1.8) (layer "F.Cu") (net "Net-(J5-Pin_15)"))
 (segment (start 135.255 41.275) (end 135.255 43.18) (width 1.8) (layer "F.Cu") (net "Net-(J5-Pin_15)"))
 (segment (start 135.255 43.18) (end 131.592006 46.842994) (width 1.8) (layer "F.Cu") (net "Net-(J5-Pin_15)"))
 (segment (start 126.365 51.435) (end 126.365 50.505988) (width 1.8) (layer "F.Cu") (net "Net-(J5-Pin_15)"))
 (segment (start 130.027994 46.842994) (end 126.365 50.505988) (width 1.8) (layer "F.Cu") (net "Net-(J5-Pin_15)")))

